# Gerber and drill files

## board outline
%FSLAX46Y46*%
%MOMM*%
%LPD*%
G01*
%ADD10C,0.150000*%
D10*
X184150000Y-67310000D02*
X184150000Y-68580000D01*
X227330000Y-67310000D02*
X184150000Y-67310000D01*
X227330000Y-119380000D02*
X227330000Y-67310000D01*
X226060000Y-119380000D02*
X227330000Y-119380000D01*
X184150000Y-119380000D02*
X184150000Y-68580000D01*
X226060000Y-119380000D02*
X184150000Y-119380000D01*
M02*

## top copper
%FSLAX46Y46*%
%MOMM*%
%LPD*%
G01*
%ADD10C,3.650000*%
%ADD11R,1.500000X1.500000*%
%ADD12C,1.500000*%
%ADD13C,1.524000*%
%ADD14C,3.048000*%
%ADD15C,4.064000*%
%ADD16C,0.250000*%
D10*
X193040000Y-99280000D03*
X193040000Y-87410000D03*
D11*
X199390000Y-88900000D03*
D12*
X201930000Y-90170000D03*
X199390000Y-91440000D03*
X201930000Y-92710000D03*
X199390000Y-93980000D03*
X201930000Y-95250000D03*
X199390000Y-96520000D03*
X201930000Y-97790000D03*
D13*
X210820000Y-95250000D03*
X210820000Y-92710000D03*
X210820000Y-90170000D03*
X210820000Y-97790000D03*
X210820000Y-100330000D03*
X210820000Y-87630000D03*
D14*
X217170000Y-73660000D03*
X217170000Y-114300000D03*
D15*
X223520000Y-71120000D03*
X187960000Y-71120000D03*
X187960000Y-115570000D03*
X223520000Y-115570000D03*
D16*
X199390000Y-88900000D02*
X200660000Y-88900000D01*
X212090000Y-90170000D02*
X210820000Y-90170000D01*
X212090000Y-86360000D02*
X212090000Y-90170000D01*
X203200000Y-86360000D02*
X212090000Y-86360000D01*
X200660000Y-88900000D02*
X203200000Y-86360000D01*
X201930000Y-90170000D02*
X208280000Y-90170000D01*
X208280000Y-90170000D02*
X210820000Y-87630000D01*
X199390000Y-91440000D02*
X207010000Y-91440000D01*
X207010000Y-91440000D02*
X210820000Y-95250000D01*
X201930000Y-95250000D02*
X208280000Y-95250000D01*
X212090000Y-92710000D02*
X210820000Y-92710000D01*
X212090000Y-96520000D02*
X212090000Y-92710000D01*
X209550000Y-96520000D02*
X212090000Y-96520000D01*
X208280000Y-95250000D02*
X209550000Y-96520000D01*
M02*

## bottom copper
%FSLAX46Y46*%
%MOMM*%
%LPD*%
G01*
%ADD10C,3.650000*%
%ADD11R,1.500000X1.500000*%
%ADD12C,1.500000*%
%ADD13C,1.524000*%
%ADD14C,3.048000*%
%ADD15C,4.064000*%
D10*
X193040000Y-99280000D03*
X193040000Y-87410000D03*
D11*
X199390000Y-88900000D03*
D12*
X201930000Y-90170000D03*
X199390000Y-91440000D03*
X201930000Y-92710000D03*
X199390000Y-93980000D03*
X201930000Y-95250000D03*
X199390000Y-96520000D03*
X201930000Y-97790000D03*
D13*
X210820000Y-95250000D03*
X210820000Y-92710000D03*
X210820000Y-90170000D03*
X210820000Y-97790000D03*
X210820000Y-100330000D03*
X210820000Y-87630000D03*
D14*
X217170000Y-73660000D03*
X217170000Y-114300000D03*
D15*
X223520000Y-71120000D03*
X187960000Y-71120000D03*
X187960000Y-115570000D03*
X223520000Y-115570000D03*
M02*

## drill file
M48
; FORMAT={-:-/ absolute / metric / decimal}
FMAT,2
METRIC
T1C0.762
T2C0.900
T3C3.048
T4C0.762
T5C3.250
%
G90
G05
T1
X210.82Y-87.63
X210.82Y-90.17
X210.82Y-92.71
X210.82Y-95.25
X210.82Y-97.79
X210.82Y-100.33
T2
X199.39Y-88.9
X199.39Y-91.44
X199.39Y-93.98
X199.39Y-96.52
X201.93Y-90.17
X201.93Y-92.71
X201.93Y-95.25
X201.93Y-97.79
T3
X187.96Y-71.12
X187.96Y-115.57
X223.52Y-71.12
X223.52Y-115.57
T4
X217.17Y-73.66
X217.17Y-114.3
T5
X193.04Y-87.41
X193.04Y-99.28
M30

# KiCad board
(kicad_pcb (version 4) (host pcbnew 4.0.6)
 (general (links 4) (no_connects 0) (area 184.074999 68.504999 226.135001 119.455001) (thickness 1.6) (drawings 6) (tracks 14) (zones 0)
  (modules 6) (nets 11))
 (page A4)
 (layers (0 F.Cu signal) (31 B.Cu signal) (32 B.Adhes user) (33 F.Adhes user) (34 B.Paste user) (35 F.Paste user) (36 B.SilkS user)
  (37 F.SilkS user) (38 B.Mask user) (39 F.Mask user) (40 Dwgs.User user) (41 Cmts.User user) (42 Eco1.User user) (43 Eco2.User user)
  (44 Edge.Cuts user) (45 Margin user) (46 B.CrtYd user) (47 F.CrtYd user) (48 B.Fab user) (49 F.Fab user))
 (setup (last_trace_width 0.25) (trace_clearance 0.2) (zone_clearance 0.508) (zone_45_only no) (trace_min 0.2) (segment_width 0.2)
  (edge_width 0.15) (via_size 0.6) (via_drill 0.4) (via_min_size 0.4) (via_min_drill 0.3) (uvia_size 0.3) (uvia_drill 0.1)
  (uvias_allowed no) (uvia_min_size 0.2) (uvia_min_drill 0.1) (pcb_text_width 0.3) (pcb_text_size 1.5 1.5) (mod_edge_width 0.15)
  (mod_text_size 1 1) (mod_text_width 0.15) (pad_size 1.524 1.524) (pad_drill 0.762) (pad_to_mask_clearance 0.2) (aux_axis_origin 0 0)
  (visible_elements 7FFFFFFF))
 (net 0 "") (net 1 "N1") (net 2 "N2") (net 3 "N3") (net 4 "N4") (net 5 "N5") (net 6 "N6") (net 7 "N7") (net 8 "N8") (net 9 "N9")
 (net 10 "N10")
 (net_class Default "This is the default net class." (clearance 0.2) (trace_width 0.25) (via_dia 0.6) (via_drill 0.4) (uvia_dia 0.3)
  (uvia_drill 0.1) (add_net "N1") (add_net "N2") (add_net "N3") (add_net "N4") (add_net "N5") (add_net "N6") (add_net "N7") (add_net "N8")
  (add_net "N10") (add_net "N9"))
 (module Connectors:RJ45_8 (layer F.Cu) (at 199.39 88.9 270)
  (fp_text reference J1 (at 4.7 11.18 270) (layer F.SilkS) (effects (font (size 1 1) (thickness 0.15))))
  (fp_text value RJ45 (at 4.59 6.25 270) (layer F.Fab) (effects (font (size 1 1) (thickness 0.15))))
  (pad Hole np_thru_hole circle (at 10.38 6.35 270) (size 3.65 3.65) (drill 3.25) (layers *.Cu *.SilkS *.Mask))
  (pad Hole np_thru_hole circle (at -1.49 6.35 270) (size 3.65 3.65) (drill 3.25) (layers *.Cu *.SilkS *.Mask))
  (pad 1 thru_hole rect (at 0 0 270) (size 1.5 1.5) (drill 0.9) (layers *.Cu *.Mask) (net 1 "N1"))
  (pad 2 thru_hole circle (at 1.27 -2.54 270) (size 1.5 1.5) (drill 0.9) (layers *.Cu *.Mask) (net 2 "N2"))
  (pad 3 thru_hole circle (at 2.54 0 270) (size 1.5 1.5) (drill 0.9) (layers *.Cu *.Mask) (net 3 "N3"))
  (pad 4 thru_hole circle (at 3.81 -2.54 270) (size 1.5 1.5) (drill 0.9) (layers *.Cu *.Mask) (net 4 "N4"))
  (pad 5 thru_hole circle (at 5.08 0 270) (size 1.5 1.5) (drill 0.9) (layers *.Cu *.Mask) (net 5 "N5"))
  (pad 6 thru_hole circle (at 6.35 -2.54 270) (size 1.5 1.5) (drill 0.9) (layers *.Cu *.Mask) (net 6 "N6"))
  (pad 7 thru_hole circle (at 7.62 0 270) (size 1.5 1.5) (drill 0.9) (layers *.Cu *.Mask) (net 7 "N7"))
  (pad 8 thru_hole circle (at 8.89 -2.54 270) (size 1.5 1.5) (drill 0.9) (layers *.Cu *.Mask) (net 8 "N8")))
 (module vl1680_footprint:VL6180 (layer F.Cu) (at 213.36 93.98)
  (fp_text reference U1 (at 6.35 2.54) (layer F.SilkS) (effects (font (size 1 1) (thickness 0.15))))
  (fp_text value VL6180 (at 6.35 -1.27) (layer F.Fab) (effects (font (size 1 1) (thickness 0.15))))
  (pad 3 thru_hole circle (at -2.54 1.27) (size 1.524 1.524) (drill 0.762) (layers *.Cu *.Mask) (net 3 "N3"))
  (pad 4 thru_hole circle (at -2.54 -1.27) (size 1.524 1.524) (drill 0.762) (layers *.Cu *.Mask) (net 6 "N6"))
  (pad 5 thru_hole circle (at -2.54 -3.81) (size 1.524 1.524) (drill 0.762) (layers *.Cu *.Mask) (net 1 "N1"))
  (pad 2 thru_hole circle (at -2.54 3.81) (size 1.524 1.524) (drill 0.762) (layers *.Cu *.Mask) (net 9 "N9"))
  (pad 1 thru_hole circle (at -2.54 6.35) (size 1.524 1.524) (drill 0.762) (layers *.Cu *.Mask) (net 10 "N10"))
  (pad 6 thru_hole circle (at -2.54 -6.35) (size 1.524 1.524) (drill 0.762) (layers *.Cu *.Mask) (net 2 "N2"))
  (pad "" np_thru_hole circle (at 3.81 -20.32) (size 3.048 3.048) (drill 0.762) (layers *.Cu *.Mask))
  (pad "" np_thru_hole circle (at 3.81 20.32) (size 3.048 3.048) (drill 0.762) (layers *.Cu *.Mask)))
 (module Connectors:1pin (layer F.Cu) (at 223.52 71.12)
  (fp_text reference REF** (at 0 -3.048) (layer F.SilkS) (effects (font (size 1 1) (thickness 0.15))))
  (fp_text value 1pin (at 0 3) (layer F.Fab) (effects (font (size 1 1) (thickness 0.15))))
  (pad 1 thru_hole circle (at 0 0) (size 4.064 4.064) (drill 3.048) (layers *.Cu *.Mask)))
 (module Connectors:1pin (layer F.Cu) (at 187.96 71.12)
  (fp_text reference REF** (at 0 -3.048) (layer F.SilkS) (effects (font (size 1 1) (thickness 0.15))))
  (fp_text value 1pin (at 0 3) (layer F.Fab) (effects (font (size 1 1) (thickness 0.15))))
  (pad 1 thru_hole circle (at 0 0) (size 4.064 4.064) (drill 3.048) (layers *.Cu *.Mask)))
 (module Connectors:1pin (layer F.Cu) (at 187.96 115.57)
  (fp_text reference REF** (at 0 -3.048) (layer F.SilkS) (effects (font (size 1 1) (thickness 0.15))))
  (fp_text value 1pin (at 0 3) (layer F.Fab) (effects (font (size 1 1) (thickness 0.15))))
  (pad 1 thru_hole circle (at 0 0) (size 4.064 4.064) (drill 3.048) (layers *.Cu *.Mask)))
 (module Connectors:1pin (layer F.Cu) (at 223.52 115.57)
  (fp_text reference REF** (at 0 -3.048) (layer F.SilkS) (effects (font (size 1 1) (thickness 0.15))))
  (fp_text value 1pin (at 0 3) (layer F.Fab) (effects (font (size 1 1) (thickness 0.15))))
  (pad 1 thru_hole circle (at 0 0) (size 4.064 4.064) (drill 3.048) (layers *.Cu *.Mask)))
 (gr_line (start 184.15 67.31) (end 184.15 68.58) (angle 90) (layer Edge.Cuts) (width 0.15))
 (gr_line (start 227.33 67.31) (end 184.15 67.31) (angle 90) (layer Edge.Cuts) (width 0.15))
 (gr_line (start 227.33 119.38) (end 227.33 67.31) (angle 90) (layer Edge.Cuts) (width 0.15))
 (gr_line (start 226.06 119.38) (end 227.33 119.38) (angle 90) (layer Edge.Cuts) (width 0.15))
 (gr_line (start 184.15 119.38) (end 184.15 68.58) (angle 90) (layer Edge.Cuts) (width 0.15))
 (gr_line (start 226.06 119.38) (end 184.15 119.38) (angle 90) (layer Edge.Cuts) (width 0.15))
 (segment (start 199.39 88.9) (end 200.66 88.9) (width 0.25) (layer F.Cu) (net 1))
 (segment (start 212.09 90.17) (end 210.82 90.17) (width 0.25) (layer F.Cu) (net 1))
 (segment (start 212.09 86.36) (end 212.09 90.17) (width 0.25) (layer F.Cu) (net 1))
 (segment (start 203.2 86.36) (end 212.09 86.36) (width 0.25) (layer F.Cu) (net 1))
 (segment (start 200.66 88.9) (end 203.2 86.36) (width 0.25) (layer F.Cu) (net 1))
 (segment (start 201.93 90.17) (end 208.28 90.17) (width 0.25) (layer F.Cu) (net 2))
 (segment (start 208.28 90.17) (end 210.82 87.63) (width 0.25) (layer F.Cu) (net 2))
 (segment (start 199.39 91.44) (end 207.01 91.44) (width 0.25) (layer F.Cu) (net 3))
 (segment (start 207.01 91.44) (end 210.82 95.25) (width 0.25) (layer F.Cu) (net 3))
 (segment (start 201.93 95.25) (end 208.28 95.25) (width 0.25) (layer F.Cu) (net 6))
 (segment (start 212.09 92.71) (end 210.82 92.71) (width 0.25) (layer F.Cu) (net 6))
 (segment (start 212.09 96.52) (end 212.09 92.71) (width 0.25) (layer F.Cu) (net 6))
 (segment (start 209.55 96.52) (end 212.09 96.52) (width 0.25) (layer F.Cu) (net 6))
 (segment (start 208.28 95.25) (end 209.55 96.52) (width 0.25) (layer F.Cu) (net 6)))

